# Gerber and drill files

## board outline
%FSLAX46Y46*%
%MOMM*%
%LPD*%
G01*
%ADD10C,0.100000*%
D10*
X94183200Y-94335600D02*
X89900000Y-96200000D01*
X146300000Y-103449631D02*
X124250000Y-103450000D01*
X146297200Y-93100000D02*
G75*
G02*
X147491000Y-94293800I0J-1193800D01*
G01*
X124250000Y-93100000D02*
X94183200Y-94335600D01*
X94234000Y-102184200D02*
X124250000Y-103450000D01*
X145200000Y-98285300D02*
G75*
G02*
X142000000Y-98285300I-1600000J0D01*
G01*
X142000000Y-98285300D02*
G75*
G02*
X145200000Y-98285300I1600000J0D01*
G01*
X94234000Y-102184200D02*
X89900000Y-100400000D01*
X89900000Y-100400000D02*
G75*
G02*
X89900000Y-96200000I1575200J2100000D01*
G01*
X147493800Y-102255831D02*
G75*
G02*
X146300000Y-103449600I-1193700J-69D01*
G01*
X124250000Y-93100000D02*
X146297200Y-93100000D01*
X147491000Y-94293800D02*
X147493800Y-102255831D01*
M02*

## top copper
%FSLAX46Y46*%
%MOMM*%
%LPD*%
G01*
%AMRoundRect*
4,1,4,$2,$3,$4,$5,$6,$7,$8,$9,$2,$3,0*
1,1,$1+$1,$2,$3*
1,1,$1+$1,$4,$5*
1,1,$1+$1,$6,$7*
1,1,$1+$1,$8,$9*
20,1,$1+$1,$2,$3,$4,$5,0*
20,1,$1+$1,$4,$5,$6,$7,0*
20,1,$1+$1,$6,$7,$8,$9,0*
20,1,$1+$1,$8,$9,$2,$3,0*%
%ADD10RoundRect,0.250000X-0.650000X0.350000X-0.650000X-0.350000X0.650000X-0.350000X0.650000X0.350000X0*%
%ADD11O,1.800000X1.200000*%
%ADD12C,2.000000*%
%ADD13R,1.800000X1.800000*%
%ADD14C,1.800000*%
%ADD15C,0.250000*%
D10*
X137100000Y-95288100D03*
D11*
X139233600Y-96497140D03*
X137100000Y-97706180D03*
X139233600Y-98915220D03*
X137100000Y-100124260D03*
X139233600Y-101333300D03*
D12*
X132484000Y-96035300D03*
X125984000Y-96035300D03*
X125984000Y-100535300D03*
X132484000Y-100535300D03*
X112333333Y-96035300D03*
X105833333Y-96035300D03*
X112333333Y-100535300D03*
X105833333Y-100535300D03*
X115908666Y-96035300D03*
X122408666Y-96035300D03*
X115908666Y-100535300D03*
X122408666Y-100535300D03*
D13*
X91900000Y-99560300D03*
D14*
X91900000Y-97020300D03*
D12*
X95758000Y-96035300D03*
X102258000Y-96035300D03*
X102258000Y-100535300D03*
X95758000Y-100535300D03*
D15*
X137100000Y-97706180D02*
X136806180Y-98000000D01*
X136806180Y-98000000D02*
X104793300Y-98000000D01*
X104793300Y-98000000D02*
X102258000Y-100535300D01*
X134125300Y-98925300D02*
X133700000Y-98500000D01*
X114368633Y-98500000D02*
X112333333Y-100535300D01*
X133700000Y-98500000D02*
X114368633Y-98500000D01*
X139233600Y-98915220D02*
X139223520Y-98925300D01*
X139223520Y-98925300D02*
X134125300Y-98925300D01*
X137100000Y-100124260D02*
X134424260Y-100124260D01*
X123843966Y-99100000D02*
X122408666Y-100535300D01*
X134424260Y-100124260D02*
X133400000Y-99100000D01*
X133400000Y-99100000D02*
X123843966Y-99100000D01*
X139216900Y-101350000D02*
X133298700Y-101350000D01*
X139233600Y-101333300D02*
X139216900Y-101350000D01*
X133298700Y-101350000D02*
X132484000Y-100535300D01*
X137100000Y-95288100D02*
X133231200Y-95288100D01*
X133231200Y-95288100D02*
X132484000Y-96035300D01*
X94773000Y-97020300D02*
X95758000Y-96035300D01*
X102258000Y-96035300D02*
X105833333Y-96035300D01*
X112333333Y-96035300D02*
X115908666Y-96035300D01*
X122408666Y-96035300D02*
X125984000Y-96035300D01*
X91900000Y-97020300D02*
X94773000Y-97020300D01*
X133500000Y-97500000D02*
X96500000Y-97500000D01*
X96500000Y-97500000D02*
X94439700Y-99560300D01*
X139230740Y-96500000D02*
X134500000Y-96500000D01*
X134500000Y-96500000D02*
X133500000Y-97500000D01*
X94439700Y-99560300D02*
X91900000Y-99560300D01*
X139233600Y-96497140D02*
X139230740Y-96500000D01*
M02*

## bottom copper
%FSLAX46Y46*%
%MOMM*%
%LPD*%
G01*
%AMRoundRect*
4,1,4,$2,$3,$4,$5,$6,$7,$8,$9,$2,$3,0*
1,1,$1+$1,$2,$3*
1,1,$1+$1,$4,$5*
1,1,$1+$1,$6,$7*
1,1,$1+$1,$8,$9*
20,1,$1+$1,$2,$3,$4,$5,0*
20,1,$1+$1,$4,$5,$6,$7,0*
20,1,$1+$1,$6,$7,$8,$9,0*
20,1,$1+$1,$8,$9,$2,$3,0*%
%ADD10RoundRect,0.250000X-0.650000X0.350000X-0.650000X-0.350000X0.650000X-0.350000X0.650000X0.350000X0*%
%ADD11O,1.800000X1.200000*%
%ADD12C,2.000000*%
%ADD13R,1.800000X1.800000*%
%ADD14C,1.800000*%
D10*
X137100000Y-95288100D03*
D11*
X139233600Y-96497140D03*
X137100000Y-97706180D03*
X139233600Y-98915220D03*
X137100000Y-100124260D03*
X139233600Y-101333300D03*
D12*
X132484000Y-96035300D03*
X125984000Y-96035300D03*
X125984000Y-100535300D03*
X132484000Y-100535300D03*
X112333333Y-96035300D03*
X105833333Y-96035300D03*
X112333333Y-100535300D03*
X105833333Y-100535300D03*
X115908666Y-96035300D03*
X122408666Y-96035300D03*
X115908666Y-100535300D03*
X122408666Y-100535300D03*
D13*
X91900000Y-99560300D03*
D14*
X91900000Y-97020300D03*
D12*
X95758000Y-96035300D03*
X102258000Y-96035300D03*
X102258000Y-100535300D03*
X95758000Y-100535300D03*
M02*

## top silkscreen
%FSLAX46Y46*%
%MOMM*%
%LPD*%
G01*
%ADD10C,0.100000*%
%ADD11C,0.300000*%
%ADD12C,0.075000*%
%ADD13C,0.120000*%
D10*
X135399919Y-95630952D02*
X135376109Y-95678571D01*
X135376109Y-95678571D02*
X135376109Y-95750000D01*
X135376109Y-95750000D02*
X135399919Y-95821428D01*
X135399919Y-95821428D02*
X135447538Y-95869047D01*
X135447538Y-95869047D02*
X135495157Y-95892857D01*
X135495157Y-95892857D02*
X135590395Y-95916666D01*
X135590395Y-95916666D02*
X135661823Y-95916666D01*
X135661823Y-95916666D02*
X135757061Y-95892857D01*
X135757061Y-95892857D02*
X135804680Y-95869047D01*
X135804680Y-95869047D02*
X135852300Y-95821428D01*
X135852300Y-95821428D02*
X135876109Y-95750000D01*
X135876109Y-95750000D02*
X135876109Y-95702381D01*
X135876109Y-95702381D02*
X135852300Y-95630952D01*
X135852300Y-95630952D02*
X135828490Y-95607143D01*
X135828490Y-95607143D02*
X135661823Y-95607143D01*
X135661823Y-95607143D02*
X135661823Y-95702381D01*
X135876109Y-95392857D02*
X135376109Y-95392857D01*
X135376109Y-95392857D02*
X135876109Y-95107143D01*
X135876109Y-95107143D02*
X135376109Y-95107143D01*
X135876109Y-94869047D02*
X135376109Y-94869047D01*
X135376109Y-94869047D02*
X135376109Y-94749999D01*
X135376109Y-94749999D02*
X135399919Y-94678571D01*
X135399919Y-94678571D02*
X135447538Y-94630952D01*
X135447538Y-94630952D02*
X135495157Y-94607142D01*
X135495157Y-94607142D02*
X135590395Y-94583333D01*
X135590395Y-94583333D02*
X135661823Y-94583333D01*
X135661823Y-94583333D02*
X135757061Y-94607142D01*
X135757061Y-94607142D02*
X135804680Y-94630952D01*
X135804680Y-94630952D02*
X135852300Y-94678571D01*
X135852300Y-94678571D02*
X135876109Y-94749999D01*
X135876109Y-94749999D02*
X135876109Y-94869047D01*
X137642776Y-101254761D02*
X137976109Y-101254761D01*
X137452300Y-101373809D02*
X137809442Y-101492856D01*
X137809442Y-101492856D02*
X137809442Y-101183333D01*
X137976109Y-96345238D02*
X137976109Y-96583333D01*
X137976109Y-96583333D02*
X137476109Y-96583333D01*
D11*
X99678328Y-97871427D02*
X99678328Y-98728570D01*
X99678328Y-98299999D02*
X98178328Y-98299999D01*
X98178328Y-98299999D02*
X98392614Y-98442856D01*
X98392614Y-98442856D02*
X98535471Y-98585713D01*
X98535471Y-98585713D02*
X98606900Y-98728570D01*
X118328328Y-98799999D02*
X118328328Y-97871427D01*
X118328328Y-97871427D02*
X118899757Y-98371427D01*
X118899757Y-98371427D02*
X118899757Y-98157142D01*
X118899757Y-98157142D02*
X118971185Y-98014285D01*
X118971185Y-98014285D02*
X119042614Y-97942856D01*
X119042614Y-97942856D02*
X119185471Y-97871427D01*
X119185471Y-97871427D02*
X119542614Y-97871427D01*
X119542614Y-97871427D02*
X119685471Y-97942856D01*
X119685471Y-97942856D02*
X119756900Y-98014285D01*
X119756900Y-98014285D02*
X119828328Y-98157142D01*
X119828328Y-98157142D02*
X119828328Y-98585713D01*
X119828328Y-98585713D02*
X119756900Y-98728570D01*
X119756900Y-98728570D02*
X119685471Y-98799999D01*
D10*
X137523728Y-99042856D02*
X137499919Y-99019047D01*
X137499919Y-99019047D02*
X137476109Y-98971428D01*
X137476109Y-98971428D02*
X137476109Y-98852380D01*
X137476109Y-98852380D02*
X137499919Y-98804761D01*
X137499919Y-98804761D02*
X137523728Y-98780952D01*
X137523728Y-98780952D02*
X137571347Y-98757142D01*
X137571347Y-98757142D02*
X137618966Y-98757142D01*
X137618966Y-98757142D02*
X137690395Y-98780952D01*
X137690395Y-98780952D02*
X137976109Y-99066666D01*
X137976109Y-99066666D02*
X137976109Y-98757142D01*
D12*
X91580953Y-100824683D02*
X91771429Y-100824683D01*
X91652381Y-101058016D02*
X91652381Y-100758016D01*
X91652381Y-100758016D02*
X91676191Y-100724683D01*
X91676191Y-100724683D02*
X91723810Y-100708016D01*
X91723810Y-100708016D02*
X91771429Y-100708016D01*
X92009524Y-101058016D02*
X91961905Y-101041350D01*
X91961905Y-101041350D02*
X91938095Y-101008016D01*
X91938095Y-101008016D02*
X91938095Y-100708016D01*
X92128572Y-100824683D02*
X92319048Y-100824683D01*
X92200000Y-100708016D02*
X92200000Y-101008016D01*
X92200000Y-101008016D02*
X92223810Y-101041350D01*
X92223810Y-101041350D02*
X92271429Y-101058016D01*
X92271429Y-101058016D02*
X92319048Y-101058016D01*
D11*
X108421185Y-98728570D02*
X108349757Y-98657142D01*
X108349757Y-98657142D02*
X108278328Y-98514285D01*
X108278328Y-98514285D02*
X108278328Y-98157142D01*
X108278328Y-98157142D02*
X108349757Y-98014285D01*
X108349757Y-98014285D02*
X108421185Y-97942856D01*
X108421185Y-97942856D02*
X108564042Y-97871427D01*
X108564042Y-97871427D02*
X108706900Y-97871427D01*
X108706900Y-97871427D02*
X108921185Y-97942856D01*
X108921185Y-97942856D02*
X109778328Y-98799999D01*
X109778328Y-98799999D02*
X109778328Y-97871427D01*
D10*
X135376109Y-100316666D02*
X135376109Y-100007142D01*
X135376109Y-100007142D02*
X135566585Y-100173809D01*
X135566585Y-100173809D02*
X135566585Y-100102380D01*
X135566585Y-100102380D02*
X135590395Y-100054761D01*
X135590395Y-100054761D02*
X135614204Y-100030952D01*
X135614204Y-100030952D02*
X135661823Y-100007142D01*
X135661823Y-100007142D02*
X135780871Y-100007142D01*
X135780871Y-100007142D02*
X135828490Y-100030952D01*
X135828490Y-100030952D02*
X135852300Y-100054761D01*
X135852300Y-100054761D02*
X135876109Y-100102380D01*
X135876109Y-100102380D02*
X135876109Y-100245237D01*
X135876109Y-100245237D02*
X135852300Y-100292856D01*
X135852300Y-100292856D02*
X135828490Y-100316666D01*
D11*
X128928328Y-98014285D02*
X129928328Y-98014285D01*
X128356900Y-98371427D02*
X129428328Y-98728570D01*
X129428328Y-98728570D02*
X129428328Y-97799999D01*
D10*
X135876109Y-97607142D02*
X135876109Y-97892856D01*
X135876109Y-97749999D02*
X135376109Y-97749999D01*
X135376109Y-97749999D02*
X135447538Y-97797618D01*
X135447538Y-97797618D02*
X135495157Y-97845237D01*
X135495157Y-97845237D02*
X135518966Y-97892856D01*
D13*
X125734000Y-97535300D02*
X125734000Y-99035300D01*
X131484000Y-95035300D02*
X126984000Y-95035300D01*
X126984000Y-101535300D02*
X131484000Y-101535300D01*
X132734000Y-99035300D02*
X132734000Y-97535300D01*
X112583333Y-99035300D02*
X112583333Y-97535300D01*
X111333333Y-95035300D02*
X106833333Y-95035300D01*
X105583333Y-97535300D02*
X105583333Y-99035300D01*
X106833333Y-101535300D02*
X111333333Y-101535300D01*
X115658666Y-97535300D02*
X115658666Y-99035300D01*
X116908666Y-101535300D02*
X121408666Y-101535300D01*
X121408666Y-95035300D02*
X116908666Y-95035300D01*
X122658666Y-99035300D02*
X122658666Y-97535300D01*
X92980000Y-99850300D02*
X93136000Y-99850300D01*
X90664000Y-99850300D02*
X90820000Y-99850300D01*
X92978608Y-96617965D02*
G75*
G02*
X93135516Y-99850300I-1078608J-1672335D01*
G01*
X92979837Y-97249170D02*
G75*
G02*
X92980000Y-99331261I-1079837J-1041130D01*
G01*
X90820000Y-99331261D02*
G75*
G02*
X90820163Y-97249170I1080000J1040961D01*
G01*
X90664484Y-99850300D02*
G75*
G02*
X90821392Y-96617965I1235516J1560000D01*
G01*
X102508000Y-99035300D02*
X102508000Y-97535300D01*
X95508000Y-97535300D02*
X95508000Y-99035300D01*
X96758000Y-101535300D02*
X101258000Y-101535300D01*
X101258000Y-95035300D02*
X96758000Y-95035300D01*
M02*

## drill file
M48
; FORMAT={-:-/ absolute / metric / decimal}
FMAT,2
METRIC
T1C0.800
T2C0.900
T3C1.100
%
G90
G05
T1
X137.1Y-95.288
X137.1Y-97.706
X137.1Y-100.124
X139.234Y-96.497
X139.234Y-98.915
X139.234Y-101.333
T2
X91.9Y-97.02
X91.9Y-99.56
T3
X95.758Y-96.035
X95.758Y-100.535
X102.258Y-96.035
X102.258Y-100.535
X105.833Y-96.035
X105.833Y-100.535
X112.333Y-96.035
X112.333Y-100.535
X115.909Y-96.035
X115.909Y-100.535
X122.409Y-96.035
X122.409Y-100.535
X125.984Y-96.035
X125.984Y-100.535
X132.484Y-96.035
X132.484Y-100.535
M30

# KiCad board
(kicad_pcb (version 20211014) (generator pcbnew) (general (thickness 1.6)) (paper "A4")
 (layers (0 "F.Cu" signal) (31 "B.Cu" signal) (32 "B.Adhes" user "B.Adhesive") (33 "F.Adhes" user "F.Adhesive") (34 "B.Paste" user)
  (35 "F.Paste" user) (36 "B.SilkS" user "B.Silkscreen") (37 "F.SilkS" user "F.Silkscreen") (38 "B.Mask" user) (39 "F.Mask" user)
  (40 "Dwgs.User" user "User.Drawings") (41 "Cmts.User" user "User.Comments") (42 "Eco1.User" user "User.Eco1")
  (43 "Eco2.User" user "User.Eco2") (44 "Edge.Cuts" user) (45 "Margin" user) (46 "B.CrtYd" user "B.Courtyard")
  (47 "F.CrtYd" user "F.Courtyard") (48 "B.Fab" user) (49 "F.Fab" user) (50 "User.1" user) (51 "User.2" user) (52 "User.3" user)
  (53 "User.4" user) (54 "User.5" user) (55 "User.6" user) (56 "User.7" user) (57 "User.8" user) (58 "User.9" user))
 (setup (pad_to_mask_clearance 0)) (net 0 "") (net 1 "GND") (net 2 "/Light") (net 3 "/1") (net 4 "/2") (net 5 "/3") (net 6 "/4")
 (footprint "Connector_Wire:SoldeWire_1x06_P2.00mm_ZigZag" (layer "F.Cu") (at 137.1 95.2881 -90)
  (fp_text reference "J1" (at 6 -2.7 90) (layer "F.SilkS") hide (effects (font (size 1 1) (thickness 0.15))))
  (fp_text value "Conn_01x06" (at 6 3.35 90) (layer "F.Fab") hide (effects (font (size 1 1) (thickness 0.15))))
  (pad "1" thru_hole roundrect (at 0 0 270) (size 1.2 1.8) (drill 0.8) (layers *.Cu *.Mask) (roundrect_rratio 0.208333) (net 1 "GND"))
  (pad "2" thru_hole oval (at 1.20904 -2.1336 270) (size 1.2 1.8) (drill 0.8) (layers *.Cu *.Mask) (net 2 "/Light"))
  (pad "3" thru_hole oval (at 2.41808 0 270) (size 1.2 1.8) (drill 0.8) (layers *.Cu *.Mask) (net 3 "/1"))
  (pad "4" thru_hole oval (at 3.62712 -2.1336 270) (size 1.2 1.8) (drill 0.8) (layers *.Cu *.Mask) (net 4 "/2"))
  (pad "5" thru_hole oval (at 4.83616 0 270) (size 1.2 1.8) (drill 0.8) (layers *.Cu *.Mask) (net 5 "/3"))
  (pad "6" thru_hole oval (at 6.0452 -2.1336 270) (size 1.2 1.8) (drill 0.8) (layers *.Cu *.Mask) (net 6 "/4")))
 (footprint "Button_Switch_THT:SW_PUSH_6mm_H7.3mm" (layer "F.Cu") (at 125.984 96.0353)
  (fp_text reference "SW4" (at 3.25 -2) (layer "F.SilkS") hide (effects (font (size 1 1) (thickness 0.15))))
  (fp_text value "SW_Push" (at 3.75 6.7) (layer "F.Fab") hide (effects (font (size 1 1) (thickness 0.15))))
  (fp_line (start -0.25 1.5) (end -0.25 3) (layer "F.SilkS") (width 0.12))
  (fp_line (start 5.5 -1) (end 1 -1) (layer "F.SilkS") (width 0.12))
  (fp_line (start 1 5.5) (end 5.5 5.5) (layer "F.SilkS") (width 0.12))
  (fp_line (start 6.75 3) (end 6.75 1.5) (layer "F.SilkS") (width 0.12))
  (pad "1" thru_hole circle (at 6.5 0 90) (size 2 2) (drill 1.1) (layers *.Cu *.Mask) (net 1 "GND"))
  (pad "1" thru_hole circle (at 0 0 90) (size 2 2) (drill 1.1) (layers *.Cu *.Mask) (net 1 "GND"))
  (pad "2" thru_hole circle (at 0 4.5 90) (size 2 2) (drill 1.1) (layers *.Cu *.Mask) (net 6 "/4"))
  (pad "2" thru_hole circle (at 6.5 4.5 90) (size 2 2) (drill 1.1) (layers *.Cu *.Mask) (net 6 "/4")))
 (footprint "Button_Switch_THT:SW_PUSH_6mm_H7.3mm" (layer "F.Cu") (at 105.833333 96.0353)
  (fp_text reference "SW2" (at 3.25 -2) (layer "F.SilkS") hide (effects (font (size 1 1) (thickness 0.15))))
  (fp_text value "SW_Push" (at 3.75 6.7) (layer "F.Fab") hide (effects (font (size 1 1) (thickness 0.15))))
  (fp_line (start 6.75 3) (end 6.75 1.5) (layer "F.SilkS") (width 0.12))
  (fp_line (start 5.5 -1) (end 1 -1) (layer "F.SilkS") (width 0.12))
  (fp_line (start -0.25 1.5) (end -0.25 3) (layer "F.SilkS") (width 0.12))
  (fp_line (start 1 5.5) (end 5.5 5.5) (layer "F.SilkS") (width 0.12))
  (pad "1" thru_hole circle (at 6.5 0 90) (size 2 2) (drill 1.1) (layers *.Cu *.Mask) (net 1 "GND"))
  (pad "1" thru_hole circle (at 0 0 90) (size 2 2) (drill 1.1) (layers *.Cu *.Mask) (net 1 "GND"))
  (pad "2" thru_hole circle (at 6.5 4.5 90) (size 2 2) (drill 1.1) (layers *.Cu *.Mask) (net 4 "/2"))
  (pad "2" thru_hole circle (at 0 4.5 90) (size 2 2) (drill 1.1) (layers *.Cu *.Mask) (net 4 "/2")))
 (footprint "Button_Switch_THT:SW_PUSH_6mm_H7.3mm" (layer "F.Cu") (at 115.908666 96.0353)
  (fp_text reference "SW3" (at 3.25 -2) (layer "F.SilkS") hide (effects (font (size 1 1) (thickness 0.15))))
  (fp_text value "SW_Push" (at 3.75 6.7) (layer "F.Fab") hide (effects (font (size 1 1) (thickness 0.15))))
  (fp_line (start -0.25 1.5) (end -0.25 3) (layer "F.SilkS") (width 0.12))
  (fp_line (start 1 5.5) (end 5.5 5.5) (layer "F.SilkS") (width 0.12))
  (fp_line (start 5.5 -1) (end 1 -1) (layer "F.SilkS") (width 0.12))
  (fp_line (start 6.75 3) (end 6.75 1.5) (layer "F.SilkS") (width 0.12))
  (pad "1" thru_hole circle (at 0 0 90) (size 2 2) (drill 1.1) (layers *.Cu *.Mask) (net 1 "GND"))
  (pad "1" thru_hole circle (at 6.5 0 90) (size 2 2) (drill 1.1) (layers *.Cu *.Mask) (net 1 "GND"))
  (pad "2" thru_hole circle (at 0 4.5 90) (size 2 2) (drill 1.1) (layers *.Cu *.Mask) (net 5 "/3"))
  (pad "2" thru_hole circle (at 6.5 4.5 90) (size 2 2) (drill 1.1) (layers *.Cu *.Mask) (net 5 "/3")))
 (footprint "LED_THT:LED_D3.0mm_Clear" (layer "F.Cu") (at 91.9 99.5603 90)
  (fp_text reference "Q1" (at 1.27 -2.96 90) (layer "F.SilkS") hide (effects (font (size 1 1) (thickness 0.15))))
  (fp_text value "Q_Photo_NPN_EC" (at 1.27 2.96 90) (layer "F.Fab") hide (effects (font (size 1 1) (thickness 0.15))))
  (fp_line (start -0.29 1.08) (end -0.29 1.236) (layer "F.SilkS") (width 0.12))
  (fp_line (start -0.29 -1.236) (end -0.29 -1.08) (layer "F.SilkS") (width 0.12))
  (fp_arc (start 2.942335 1.078608) (mid 1.366487 1.987659) (end -0.29 1.235516) (layer "F.SilkS") (width 0.12))
  (fp_arc (start 2.31113 1.079837) (mid 1.270117 1.5) (end 0.229039 1.08) (layer "F.SilkS") (width 0.12))
  (fp_arc (start 0.229039 -1.08) (mid 1.270117 -1.5) (end 2.31113 -1.079837) (layer "F.SilkS") (width 0.12))
  (fp_arc (start -0.29 -1.235516) (mid 1.366487 -1.987659) (end 2.942335 -1.078608) (layer "F.SilkS") (width 0.12))
  (pad "1" thru_hole rect (at 0 0 90) (size 1.8 1.8) (drill 0.9) (layers *.Cu *.Mask) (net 2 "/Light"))
  (pad "2" thru_hole circle (at 2.54 0 90) (size 1.8 1.8) (drill 0.9) (layers *.Cu *.Mask) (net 1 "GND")))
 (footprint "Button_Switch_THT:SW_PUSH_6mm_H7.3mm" (layer "F.Cu") (at 95.758 96.0353)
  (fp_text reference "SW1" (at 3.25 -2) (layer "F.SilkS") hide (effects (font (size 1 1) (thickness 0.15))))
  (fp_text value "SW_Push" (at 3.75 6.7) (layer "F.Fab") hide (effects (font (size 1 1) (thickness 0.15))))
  (fp_line (start 6.75 3) (end 6.75 1.5) (layer "F.SilkS") (width 0.12))
  (fp_line (start -0.25 1.5) (end -0.25 3) (layer "F.SilkS") (width 0.12))
  (fp_line (start 1 5.5) (end 5.5 5.5) (layer "F.SilkS") (width 0.12))
  (fp_line (start 5.5 -1) (end 1 -1) (layer "F.SilkS") (width 0.12))
  (pad "1" thru_hole circle (at 0 0 90) (size 2 2) (drill 1.1) (layers *.Cu *.Mask) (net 1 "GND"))
  (pad "1" thru_hole circle (at 6.5 0 90) (size 2 2) (drill 1.1) (layers *.Cu *.Mask) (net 1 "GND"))
  (pad "2" thru_hole circle (at 6.5 4.5 90) (size 2 2) (drill 1.1) (layers *.Cu *.Mask) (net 3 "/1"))
  (pad "2" thru_hole circle (at 0 4.5 90) (size 2 2) (drill 1.1) (layers *.Cu *.Mask) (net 3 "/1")))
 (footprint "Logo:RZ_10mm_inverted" (layer "B.Cu") (at 129.3368 98.2472 180)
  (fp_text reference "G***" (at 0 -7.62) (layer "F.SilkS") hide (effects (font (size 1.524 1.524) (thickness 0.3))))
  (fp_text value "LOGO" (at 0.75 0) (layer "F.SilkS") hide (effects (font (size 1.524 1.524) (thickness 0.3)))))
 (gr_line (start 94.1832 94.3356) (end 89.9 96.2) (layer "Edge.Cuts") (width 0.1))
 (gr_line (start 146.3 103.449631) (end 124.25 103.45) (layer "Edge.Cuts") (width 0.1))
 (gr_arc (start 146.2972 93.1) (mid 147.141344 93.449656) (end 147.491 94.2938) (layer "Edge.Cuts") (width 0.1))
 (gr_line (start 124.25 93.1) (end 94.1832 94.3356) (layer "Edge.Cuts") (width 0.1))
 (gr_line (start 94.234 102.1842) (end 124.25 103.45) (layer "Edge.Cuts") (width 0.1))
 (gr_circle (center 143.6 98.2853) (end 145.2 98.2853) (layer "Edge.Cuts") (width 0.1) (fill none))
 (gr_line (start 94.234 102.1842) (end 89.9 100.4) (layer "Edge.Cuts") (width 0.1))
 (gr_arc (start 89.9 100.4) (mid 88.850082 98.3) (end 89.9 96.2) (layer "Edge.Cuts") (width 0.1))
 (gr_arc (start 147.4938 102.255831) (mid 147.144173 103.100004) (end 146.3 103.449631) (layer "Edge.Cuts") (width 0.1))
 (gr_line (start 124.25 93.1) (end 146.2972 93.1) (layer "Edge.Cuts") (width 0.1))
 (gr_line (start 147.491 94.2938) (end 147.4938 102.255831) (layer "Edge.Cuts") (width 0.1))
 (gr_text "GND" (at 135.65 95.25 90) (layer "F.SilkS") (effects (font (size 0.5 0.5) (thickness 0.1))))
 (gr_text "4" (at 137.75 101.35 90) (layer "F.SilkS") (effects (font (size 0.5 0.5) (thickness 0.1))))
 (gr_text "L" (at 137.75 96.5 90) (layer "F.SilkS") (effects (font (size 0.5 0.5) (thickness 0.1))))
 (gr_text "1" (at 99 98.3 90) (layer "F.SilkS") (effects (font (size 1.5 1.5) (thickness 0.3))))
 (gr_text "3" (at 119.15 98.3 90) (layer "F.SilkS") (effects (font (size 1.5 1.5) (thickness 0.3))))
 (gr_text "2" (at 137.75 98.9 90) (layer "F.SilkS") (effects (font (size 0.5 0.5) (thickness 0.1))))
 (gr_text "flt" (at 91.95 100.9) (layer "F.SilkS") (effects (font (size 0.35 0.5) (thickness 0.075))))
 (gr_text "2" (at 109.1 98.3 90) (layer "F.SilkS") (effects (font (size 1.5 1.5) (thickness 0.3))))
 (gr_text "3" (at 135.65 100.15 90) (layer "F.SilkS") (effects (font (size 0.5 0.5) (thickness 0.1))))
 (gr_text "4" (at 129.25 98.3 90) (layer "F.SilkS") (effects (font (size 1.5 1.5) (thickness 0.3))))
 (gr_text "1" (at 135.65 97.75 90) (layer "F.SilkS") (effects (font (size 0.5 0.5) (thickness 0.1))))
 (segment (start 137.1 97.70618) (end 136.80618 98) (width 0.25) (layer "F.Cu") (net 3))
 (segment (start 136.80618 98) (end 104.7933 98) (width 0.25) (layer "F.Cu") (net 3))
 (segment (start 104.7933 98) (end 102.258 100.5353) (width 0.25) (layer "F.Cu") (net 3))
 (segment (start 134.1253 98.9253) (end 133.7 98.5) (width 0.25) (layer "F.Cu") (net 4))
 (segment (start 114.368633 98.5) (end 112.333333 100.5353) (width 0.25) (layer "F.Cu") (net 4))
 (segment (start 133.7 98.5) (end 114.368633 98.5) (width 0.25) (layer "F.Cu") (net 4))
 (segment (start 139.2336 98.91522) (end 139.22352 98.9253) (width 0.25) (layer "F.Cu") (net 4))
 (segment (start 139.22352 98.9253) (end 134.1253 98.9253) (width 0.25) (layer "F.Cu") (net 4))
 (segment (start 137.1 100.12426) (end 134.42426 100.12426) (width 0.25) (layer "F.Cu") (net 5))
 (segment (start 123.843966 99.1) (end 122.408666 100.5353) (width 0.25) (layer "F.Cu") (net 5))
 (segment (start 134.42426 100.12426) (end 133.4 99.1) (width 0.25) (layer "F.Cu") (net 5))
 (segment (start 133.4 99.1) (end 123.843966 99.1) (width 0.25) (layer "F.Cu") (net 5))
 (segment (start 139.2169 101.35) (end 133.2987 101.35) (width 0.25) (layer "F.Cu") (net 6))
 (segment (start 139.2336 101.3333) (end 139.2169 101.35) (width 0.25) (layer "F.Cu") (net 6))
 (segment (start 133.2987 101.35) (end 132.484 100.5353) (width 0.25) (layer "F.Cu") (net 6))
 (segment (start 137.1 95.2881) (end 133.2312 95.2881) (width 0.25) (layer "F.Cu") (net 1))
 (segment (start 133.2312 95.2881) (end 132.484 96.0353) (width 0.25) (layer "F.Cu") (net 1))
 (segment (start 94.773 97.0203) (end 95.758 96.0353) (width 0.25) (layer "F.Cu") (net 1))
 (segment (start 102.258 96.0353) (end 105.833333 96.0353) (width 0.25) (layer "F.Cu") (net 1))
 (segment (start 112.333333 96.0353) (end 115.908666 96.0353) (width 0.25) (layer "F.Cu") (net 1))
 (segment (start 122.408666 96.0353) (end 125.984 96.0353) (width 0.25) (layer "F.Cu") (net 1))
 (segment (start 91.9 97.0203) (end 94.773 97.0203) (width 0.25) (layer "F.Cu") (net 1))
 (segment (start 133.5 97.5) (end 96.5 97.5) (width 0.25) (layer "F.Cu") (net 2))
 (segment (start 96.5 97.5) (end 94.4397 99.5603) (width 0.25) (layer "F.Cu") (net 2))
 (segment (start 139.23074 96.5) (end 134.5 96.5) (width 0.25) (layer "F.Cu") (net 2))
 (segment (start 134.5 96.5) (end 133.5 97.5) (width 0.25) (layer "F.Cu") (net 2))
 (segment (start 94.4397 99.5603) (end 91.9 99.5603) (width 0.25) (layer "F.Cu") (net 2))
 (segment (start 139.2336 96.49714) (end 139.23074 96.5) (width 0.25) (layer "F.Cu") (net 2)))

